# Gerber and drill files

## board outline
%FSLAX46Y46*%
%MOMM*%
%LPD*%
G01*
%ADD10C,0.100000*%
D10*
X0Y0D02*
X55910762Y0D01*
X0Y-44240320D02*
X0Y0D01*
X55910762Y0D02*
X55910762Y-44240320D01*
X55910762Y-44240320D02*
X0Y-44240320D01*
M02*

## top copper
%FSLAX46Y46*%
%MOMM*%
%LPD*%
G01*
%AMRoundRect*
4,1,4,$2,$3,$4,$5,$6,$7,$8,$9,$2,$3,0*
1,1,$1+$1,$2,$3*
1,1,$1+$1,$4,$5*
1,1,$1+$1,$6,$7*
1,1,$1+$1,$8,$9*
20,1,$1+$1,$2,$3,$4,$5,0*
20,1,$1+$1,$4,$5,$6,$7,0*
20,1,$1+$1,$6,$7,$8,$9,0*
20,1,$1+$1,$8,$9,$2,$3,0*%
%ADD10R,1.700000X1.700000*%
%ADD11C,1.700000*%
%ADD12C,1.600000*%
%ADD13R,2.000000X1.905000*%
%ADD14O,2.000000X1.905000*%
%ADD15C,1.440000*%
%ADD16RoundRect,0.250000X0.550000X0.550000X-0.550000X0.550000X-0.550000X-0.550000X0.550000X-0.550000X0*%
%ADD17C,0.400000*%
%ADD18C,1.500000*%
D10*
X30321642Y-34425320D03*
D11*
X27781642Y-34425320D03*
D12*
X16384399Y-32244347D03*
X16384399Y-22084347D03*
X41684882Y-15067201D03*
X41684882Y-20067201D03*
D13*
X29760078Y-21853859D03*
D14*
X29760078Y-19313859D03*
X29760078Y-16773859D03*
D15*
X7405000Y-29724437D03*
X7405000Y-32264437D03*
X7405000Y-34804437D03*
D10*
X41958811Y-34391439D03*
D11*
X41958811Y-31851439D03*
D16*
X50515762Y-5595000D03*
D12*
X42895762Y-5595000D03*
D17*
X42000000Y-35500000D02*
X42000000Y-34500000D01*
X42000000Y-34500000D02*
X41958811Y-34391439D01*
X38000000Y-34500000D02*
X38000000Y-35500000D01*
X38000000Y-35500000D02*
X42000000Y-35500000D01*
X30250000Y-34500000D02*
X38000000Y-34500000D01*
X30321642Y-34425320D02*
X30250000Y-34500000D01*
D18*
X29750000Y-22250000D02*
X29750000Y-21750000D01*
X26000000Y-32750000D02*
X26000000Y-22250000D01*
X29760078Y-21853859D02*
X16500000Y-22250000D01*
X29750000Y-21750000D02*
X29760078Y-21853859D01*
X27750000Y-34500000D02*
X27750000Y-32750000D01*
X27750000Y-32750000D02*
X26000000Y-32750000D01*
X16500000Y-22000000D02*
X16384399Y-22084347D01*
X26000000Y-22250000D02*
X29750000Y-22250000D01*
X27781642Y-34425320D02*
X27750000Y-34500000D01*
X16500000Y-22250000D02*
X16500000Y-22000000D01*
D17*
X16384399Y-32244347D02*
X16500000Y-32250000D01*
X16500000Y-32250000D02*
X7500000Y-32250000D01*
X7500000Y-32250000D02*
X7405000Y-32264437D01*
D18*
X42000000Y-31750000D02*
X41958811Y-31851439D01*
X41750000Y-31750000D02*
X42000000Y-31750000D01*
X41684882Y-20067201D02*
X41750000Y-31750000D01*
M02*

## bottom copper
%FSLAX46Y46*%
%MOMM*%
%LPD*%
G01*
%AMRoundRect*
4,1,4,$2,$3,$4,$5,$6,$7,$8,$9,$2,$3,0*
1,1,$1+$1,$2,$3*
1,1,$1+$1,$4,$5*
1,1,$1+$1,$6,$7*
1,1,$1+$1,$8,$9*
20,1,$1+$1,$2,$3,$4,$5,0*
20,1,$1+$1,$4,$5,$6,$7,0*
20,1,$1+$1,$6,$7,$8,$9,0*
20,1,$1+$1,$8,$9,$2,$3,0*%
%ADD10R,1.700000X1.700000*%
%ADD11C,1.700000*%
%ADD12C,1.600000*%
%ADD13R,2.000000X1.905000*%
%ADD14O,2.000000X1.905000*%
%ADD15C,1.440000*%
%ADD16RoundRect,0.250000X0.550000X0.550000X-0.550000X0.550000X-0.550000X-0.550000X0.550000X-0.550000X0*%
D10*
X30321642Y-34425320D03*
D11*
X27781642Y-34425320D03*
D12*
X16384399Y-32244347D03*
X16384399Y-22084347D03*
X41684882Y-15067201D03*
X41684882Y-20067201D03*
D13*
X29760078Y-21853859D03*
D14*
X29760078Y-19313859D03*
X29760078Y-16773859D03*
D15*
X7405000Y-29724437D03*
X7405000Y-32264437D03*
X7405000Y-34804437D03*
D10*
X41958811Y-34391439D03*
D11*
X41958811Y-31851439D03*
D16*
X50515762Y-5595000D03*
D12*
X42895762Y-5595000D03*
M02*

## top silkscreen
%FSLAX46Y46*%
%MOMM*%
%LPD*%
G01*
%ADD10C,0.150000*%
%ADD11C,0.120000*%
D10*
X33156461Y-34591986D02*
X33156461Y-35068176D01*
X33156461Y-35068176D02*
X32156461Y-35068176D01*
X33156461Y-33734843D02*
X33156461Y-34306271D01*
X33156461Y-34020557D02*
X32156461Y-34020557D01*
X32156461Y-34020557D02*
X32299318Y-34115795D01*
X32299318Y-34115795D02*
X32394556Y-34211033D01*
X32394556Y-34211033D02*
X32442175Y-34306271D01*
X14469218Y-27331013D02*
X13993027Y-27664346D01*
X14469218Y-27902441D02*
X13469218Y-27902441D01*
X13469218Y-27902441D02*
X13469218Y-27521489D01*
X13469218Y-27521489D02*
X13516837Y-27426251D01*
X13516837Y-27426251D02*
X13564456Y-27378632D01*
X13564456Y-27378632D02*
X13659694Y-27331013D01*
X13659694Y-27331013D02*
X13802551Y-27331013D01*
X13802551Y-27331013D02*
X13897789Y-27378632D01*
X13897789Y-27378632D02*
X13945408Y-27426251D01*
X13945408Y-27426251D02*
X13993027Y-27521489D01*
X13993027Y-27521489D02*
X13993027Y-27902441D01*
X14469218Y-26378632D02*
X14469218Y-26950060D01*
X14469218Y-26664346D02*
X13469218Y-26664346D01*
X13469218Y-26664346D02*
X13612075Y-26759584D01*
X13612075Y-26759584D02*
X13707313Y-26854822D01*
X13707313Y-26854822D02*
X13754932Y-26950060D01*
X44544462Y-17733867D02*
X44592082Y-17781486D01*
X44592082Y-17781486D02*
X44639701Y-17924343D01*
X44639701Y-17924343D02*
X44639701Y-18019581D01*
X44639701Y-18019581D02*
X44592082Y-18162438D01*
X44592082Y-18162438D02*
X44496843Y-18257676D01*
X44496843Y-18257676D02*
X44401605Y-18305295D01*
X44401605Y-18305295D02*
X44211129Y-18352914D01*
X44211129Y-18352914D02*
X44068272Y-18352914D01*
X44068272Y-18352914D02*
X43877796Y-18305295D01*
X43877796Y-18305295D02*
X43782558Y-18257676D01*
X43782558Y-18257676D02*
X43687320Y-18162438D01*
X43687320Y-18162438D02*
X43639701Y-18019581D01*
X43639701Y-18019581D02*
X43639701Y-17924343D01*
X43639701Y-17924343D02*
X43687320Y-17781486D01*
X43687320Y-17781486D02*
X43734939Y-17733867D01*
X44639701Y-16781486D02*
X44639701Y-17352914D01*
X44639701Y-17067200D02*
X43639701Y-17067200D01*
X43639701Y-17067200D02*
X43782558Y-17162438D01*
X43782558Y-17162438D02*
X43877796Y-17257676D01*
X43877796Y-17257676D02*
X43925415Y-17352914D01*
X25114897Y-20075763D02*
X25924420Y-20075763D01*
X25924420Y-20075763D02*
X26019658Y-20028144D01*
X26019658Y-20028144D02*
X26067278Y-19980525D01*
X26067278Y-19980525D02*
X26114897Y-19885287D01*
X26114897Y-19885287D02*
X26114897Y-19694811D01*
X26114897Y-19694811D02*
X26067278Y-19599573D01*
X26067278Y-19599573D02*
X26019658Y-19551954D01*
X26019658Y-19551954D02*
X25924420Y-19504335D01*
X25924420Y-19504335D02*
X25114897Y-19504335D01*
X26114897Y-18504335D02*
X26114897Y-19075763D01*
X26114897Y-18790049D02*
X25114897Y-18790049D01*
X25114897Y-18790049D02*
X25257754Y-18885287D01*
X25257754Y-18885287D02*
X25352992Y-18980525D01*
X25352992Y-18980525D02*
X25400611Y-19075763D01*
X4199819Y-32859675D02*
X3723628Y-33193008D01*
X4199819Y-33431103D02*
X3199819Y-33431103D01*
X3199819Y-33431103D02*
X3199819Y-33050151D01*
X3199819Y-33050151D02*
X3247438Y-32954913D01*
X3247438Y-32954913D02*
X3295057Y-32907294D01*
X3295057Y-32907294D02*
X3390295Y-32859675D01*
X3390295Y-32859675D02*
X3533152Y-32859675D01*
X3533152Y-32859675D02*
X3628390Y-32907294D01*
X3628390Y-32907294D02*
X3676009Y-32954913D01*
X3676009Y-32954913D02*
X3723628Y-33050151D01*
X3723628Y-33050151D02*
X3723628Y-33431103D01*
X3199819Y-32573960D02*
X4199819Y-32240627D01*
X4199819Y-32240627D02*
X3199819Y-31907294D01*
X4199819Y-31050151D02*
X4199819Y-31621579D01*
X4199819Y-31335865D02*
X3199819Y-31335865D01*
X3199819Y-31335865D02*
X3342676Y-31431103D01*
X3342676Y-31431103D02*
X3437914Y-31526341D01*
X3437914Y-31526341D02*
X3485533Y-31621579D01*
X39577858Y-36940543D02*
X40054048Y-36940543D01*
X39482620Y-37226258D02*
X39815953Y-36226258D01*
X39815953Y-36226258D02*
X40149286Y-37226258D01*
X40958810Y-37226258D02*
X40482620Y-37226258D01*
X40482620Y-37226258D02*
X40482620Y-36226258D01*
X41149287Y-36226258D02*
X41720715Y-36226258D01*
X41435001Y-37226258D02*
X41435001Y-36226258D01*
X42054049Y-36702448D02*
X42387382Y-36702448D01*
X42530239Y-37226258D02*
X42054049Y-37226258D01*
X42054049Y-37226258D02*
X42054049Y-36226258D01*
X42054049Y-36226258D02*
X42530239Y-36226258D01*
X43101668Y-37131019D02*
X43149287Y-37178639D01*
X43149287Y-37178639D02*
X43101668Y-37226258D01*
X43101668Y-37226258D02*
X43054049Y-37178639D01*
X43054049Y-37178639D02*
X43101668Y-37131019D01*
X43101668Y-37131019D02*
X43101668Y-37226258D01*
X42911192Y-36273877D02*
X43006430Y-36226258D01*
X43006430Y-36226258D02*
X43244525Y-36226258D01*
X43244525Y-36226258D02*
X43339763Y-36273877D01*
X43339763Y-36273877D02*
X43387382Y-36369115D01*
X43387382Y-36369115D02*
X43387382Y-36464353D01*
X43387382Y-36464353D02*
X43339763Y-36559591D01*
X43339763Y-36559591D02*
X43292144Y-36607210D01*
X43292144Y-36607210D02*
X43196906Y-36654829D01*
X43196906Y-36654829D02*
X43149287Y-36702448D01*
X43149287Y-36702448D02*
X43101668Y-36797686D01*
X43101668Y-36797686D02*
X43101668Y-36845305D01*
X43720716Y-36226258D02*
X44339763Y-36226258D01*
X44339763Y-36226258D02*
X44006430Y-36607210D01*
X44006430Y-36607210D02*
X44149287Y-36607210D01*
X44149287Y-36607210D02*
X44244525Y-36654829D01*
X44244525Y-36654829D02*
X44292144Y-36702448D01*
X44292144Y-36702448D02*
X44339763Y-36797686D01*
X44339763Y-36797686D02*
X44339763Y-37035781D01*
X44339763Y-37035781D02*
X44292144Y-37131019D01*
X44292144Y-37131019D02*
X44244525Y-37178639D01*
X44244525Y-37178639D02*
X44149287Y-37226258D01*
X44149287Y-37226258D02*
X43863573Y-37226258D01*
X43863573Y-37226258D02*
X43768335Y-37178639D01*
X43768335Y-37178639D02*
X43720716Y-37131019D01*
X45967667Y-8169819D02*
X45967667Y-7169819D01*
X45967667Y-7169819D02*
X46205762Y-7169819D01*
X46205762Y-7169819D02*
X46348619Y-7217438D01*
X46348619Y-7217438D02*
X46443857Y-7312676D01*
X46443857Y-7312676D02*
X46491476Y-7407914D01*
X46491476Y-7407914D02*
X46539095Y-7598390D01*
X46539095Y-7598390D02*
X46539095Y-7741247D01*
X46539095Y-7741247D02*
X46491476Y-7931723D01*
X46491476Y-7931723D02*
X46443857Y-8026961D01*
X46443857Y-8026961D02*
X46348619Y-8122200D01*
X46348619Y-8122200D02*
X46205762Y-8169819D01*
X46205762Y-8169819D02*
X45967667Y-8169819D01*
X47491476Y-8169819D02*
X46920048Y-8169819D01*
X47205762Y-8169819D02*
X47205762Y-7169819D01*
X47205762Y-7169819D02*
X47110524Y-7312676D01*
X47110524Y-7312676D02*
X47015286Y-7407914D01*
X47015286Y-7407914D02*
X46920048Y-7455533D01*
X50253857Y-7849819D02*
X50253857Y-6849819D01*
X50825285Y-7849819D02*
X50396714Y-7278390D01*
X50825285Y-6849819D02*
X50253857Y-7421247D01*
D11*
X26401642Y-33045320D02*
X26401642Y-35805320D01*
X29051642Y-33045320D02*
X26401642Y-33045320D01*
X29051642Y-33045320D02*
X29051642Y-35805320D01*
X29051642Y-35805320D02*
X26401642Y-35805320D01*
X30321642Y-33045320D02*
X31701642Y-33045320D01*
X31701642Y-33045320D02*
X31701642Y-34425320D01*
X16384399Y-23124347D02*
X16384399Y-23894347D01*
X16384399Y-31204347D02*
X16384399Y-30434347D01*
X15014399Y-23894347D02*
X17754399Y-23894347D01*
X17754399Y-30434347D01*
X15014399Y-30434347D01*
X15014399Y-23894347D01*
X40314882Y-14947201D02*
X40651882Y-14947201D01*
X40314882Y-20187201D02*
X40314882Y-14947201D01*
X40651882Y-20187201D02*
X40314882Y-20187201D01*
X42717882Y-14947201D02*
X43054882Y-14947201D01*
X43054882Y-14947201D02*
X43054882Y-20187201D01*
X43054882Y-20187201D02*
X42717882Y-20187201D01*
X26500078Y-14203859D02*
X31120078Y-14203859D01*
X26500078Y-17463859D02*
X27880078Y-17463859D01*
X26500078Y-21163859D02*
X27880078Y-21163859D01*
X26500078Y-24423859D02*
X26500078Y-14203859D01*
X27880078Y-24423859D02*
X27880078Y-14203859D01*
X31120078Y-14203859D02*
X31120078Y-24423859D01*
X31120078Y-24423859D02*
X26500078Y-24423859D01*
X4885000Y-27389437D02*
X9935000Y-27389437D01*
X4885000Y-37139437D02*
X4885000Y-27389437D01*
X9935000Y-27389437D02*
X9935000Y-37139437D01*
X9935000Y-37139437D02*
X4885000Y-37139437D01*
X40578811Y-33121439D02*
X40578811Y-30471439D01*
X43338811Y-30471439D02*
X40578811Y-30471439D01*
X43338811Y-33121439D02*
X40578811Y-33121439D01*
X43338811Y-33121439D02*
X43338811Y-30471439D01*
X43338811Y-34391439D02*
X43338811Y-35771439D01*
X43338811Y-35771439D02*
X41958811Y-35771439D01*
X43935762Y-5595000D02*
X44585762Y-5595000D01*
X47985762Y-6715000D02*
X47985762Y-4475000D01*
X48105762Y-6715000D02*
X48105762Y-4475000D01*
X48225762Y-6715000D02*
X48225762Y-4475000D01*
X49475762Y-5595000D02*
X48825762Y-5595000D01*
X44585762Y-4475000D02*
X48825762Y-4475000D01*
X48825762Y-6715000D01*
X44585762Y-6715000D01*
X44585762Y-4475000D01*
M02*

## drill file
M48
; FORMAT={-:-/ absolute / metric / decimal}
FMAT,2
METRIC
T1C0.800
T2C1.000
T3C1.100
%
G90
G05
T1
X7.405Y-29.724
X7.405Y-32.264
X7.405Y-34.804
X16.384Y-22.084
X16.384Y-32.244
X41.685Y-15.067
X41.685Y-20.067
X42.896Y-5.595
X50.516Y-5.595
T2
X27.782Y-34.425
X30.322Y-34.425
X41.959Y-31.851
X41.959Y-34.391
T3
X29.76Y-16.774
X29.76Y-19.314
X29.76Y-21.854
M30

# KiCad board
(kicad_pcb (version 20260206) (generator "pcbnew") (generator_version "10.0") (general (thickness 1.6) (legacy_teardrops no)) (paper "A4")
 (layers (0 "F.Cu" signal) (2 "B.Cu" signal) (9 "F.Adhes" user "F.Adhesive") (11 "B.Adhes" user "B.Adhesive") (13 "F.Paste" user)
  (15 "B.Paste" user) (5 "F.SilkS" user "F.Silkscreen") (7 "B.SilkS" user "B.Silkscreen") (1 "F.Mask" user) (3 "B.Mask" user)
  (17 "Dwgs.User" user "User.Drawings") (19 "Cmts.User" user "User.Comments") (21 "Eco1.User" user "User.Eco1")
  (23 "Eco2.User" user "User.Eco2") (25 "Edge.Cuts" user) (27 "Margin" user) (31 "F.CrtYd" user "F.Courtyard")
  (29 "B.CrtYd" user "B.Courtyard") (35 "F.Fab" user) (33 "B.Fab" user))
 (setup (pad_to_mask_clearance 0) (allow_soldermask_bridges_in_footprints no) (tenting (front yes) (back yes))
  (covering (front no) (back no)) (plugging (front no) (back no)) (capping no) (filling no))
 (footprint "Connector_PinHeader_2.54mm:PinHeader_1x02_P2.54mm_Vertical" (layer "F.Cu") (at 30.321642 34.42532 -90)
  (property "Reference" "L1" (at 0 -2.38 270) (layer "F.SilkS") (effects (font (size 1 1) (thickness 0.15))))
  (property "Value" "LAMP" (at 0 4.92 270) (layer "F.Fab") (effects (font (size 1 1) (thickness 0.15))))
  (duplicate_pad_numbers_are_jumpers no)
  (fp_line (start -1.38 3.92) (end 1.38 3.92) (stroke (width 0.12) (type solid)) (layer "F.SilkS"))
  (fp_line (start -1.38 1.27) (end -1.38 3.92) (stroke (width 0.12) (type solid)) (layer "F.SilkS"))
  (fp_line (start -1.38 1.27) (end 1.38 1.27) (stroke (width 0.12) (type solid)) (layer "F.SilkS"))
  (fp_line (start 1.38 1.27) (end 1.38 3.92) (stroke (width 0.12) (type solid)) (layer "F.SilkS"))
  (fp_line (start -1.38 0) (end -1.38 -1.38) (stroke (width 0.12) (type solid)) (layer "F.SilkS"))
  (fp_line (start -1.38 -1.38) (end 0 -1.38) (stroke (width 0.12) (type solid)) (layer "F.SilkS"))
  (pad "1" thru_hole rect (at 0 0 270) (size 1.7 1.7) (drill 1) (layers "*.Cu" "*.Mask") (remove_unused_layers no) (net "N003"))
  (pad "2" thru_hole circle (at 0 2.54 270) (size 1.7 1.7) (drill 1) (layers "*.Cu" "*.Mask") (remove_unused_layers no) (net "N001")))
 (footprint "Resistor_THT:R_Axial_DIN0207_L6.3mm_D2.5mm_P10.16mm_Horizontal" (layer "F.Cu") (at 16.384399 32.244347 90)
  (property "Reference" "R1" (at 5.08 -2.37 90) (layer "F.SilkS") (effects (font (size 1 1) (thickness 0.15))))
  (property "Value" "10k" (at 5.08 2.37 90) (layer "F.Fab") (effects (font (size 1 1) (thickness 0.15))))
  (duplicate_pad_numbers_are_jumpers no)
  (fp_line (start 9.12 0) (end 8.35 0) (stroke (width 0.12) (type solid)) (layer "F.SilkS"))
  (fp_line (start 1.04 0) (end 1.81 0) (stroke (width 0.12) (type solid)) (layer "F.SilkS"))
  (fp_rect (start 1.81 -1.37) (end 8.35 1.37) (stroke (width 0.12) (type solid)) (fill no) (layer "F.SilkS"))
  (pad "1" thru_hole circle (at 0 0 90) (size 1.6 1.6) (drill 0.8) (layers "*.Cu" "*.Mask") (remove_unused_layers no) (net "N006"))
  (pad "2" thru_hole circle (at 10.16 0 90) (size 1.6 1.6) (drill 0.8) (layers "*.Cu" "*.Mask") (remove_unused_layers no) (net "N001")))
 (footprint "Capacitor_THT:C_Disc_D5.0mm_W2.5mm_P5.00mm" (layer "F.Cu") (at 41.684882 15.067201 -90)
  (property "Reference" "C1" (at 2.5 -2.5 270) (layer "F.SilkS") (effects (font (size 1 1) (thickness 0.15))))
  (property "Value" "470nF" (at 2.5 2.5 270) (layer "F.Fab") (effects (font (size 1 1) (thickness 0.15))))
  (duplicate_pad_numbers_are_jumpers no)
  (fp_line (start -0.12 1.37) (end -0.12 1.033) (stroke (width 0.12) (type solid)) (layer "F.SilkS"))
  (fp_line (start 5.12 1.37) (end -0.12 1.37) (stroke (width 0.12) (type solid)) (layer "F.SilkS"))
  (fp_line (start 5.12 1.033) (end 5.12 1.37) (stroke (width 0.12) (type solid)) (layer "F.SilkS"))
  (fp_line (start -0.12 -1.033) (end -0.12 -1.37) (stroke (width 0.12) (type solid)) (layer "F.SilkS"))
  (fp_line (start -0.12 -1.37) (end 5.12 -1.37) (stroke (width 0.12) (type solid)) (layer "F.SilkS"))
  (fp_line (start 5.12 -1.37) (end 5.12 -1.033) (stroke (width 0.12) (type solid)) (layer "F.SilkS"))
  (pad "1" thru_hole circle (at 0 0 270) (size 1.6 1.6) (drill 0.8) (layers "*.Cu" "*.Mask") (remove_unused_layers no))
  (pad "2" thru_hole circle (at 5 0 270) (size 1.6 1.6) (drill 0.8) (layers "*.Cu" "*.Mask") (remove_unused_layers no) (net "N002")))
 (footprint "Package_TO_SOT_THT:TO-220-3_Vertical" (layer "F.Cu") (at 29.760078 21.853859 90)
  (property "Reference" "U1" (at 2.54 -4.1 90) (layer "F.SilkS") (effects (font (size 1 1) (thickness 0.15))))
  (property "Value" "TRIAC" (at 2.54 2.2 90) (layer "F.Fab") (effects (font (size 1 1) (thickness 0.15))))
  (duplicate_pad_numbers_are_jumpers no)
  (fp_line (start 7.65 -3.26) (end 7.65 1.36) (stroke (width 0.12) (type solid)) (layer "F.SilkS"))
  (fp_line (start 4.39 -3.26) (end 4.39 -1.88) (stroke (width 0.12) (type solid)) (layer "F.SilkS"))
  (fp_line (start 0.69 -3.26) (end 0.69 -1.88) (stroke (width 0.12) (type solid)) (layer "F.SilkS"))
  (fp_line (start -2.57 -3.26) (end 7.65 -3.26) (stroke (width 0.12) (type solid)) (layer "F.SilkS"))
  (fp_line (start -2.57 -1.88) (end 7.65 -1.88) (stroke (width 0.12) (type solid)) (layer "F.SilkS"))
  (fp_line (start 7.65 1.36) (end -2.57 1.36) (stroke (width 0.12) (type solid)) (layer "F.SilkS"))
  (fp_line (start -2.57 1.36) (end -2.57 -3.26) (stroke (width 0.12) (type solid)) (layer "F.SilkS"))
  (pad "1" thru_hole rect (at 0 0 90) (size 1.905 2) (drill 1.1) (layers "*.Cu" "*.Mask") (remove_unused_layers no) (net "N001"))
  (pad "2" thru_hole oval (at 2.54 0 90) (size 1.905 2) (drill 1.1) (layers "*.Cu" "*.Mask") (remove_unused_layers no) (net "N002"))
  (pad "3" thru_hole oval (at 5.08 0 90) (size 1.905 2) (drill 1.1) (layers "*.Cu" "*.Mask") (remove_unused_layers no) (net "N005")))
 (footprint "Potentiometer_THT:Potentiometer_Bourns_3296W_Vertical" (layer "F.Cu") (at 7.405 29.724437 90)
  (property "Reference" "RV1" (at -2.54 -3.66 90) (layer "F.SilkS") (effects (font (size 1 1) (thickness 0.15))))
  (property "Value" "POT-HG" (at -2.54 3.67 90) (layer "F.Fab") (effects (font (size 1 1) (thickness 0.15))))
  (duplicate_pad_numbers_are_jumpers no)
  (fp_line (start 2.335 -2.52) (end 2.335 2.53) (stroke (width 0.12) (type solid)) (layer "F.SilkS"))
  (fp_line (start -7.415 -2.52) (end 2.335 -2.52) (stroke (width 0.12) (type solid)) (layer "F.SilkS"))
  (fp_line (start 2.335 2.53) (end -7.415 2.53) (stroke (width 0.12) (type solid)) (layer "F.SilkS"))
  (fp_line (start -7.415 2.53) (end -7.415 -2.52) (stroke (width 0.12) (type solid)) (layer "F.SilkS"))
  (pad "1" thru_hole circle (at 0 0 90) (size 1.44 1.44) (drill 0.8) (layers "*.Cu" "*.Mask") (remove_unused_layers no) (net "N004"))
  (pad "2" thru_hole circle (at -2.54 0 90) (size 1.44 1.44) (drill 0.8) (layers "*.Cu" "*.Mask") (remove_unused_layers no) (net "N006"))
  (pad "3" thru_hole circle (at -5.08 0 90) (size 1.44 1.44) (drill 0.8) (layers "*.Cu" "*.Mask") (remove_unused_layers no)))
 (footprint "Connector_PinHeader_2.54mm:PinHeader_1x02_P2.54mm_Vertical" (layer "F.Cu") (at 41.958811 34.391439 180)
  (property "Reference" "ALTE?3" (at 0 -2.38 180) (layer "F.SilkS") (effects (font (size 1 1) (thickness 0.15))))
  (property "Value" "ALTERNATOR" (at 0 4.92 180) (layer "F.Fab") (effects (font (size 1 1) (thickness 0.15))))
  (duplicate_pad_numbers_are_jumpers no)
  (fp_line (start 1.38 1.27) (end 1.38 3.92) (stroke (width 0.12) (type solid)) (layer "F.SilkS"))
  (fp_line (start -1.38 3.92) (end 1.38 3.92) (stroke (width 0.12) (type solid)) (layer "F.SilkS"))
  (fp_line (start -1.38 1.27) (end 1.38 1.27) (stroke (width 0.12) (type solid)) (layer "F.SilkS"))
  (fp_line (start -1.38 1.27) (end -1.38 3.92) (stroke (width 0.12) (type solid)) (layer "F.SilkS"))
  (fp_line (start -1.38 0) (end -1.38 -1.38) (stroke (width 0.12) (type solid)) (layer "F.SilkS"))
  (fp_line (start -1.38 -1.38) (end 0 -1.38) (stroke (width 0.12) (type solid)) (layer "F.SilkS"))
  (pad "1" thru_hole rect (at 0 0 180) (size 1.7 1.7) (drill 1) (layers "*.Cu" "*.Mask") (remove_unused_layers no) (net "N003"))
  (pad "2" thru_hole circle (at 0 2.54 180) (size 1.7 1.7) (drill 1) (layers "*.Cu" "*.Mask") (remove_unused_layers no) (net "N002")))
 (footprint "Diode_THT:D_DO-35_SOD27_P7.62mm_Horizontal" (layer "F.Cu") (at 50.515762 5.595 180)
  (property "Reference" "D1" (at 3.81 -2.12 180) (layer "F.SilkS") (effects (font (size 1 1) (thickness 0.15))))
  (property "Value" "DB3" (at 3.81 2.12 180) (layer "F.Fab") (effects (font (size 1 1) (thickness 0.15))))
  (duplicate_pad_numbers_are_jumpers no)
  (fp_line (start 6.58 0) (end 5.93 0) (stroke (width 0.12) (type solid)) (layer "F.SilkS"))
  (fp_line (start 2.53 -1.12) (end 2.53 1.12) (stroke (width 0.12) (type solid)) (layer "F.SilkS"))
  (fp_line (start 2.41 -1.12) (end 2.41 1.12) (stroke (width 0.12) (type solid)) (layer "F.SilkS"))
  (fp_line (start 2.29 -1.12) (end 2.29 1.12) (stroke (width 0.12) (type solid)) (layer "F.SilkS"))
  (fp_line (start 1.04 0) (end 1.69 0) (stroke (width 0.12) (type solid)) (layer "F.SilkS"))
  (fp_rect (start 1.69 -1.12) (end 5.93 1.12) (stroke (width 0.12) (type solid)) (fill no) (layer "F.SilkS"))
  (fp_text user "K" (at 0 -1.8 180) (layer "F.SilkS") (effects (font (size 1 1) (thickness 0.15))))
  (pad "1" thru_hole roundrect (at 0 0 180) (size 1.6 1.6) (drill 0.8) (layers "*.Cu" "*.Mask") (remove_unused_layers no)
   (roundrect_rratio 0.15625))
  (pad "2" thru_hole circle (at 7.62 0 180) (size 1.6 1.6) (drill 0.8) (layers "*.Cu" "*.Mask") (remove_unused_layers no)))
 (gr_line (start 0 0) (end 55.910762 0) (stroke (width 0.1) (type default)) (layer "Edge.Cuts"))
 (gr_line (start 0 44.24032) (end 0 0) (stroke (width 0.1) (type default)) (layer "Edge.Cuts"))
 (gr_line (start 55.910762 0) (end 55.910762 44.24032) (stroke (width 0.1) (type default)) (layer "Edge.Cuts"))
 (gr_line (start 55.910762 44.24032) (end 0 44.24032) (stroke (width 0.1) (type default)) (layer "Edge.Cuts"))
 (segment (start 42 35.5) (end 42 34.5) (width 0.4) (layer "F.Cu") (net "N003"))
 (segment (start 42 34.5) (end 41.958811 34.391439) (width 0.4) (layer "F.Cu") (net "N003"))
 (segment (start 38 34.5) (end 38 35.5) (width 0.4) (layer "F.Cu") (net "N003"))
 (segment (start 38 35.5) (end 42 35.5) (width 0.4) (layer "F.Cu") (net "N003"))
 (segment (start 30.25 34.5) (end 38 34.5) (width 0.4) (layer "F.Cu") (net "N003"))
 (segment (start 30.321642 34.42532) (end 30.25 34.5) (width 0.4) (layer "F.Cu") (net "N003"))
 (segment (start 29.75 22.25) (end 29.75 21.75) (width 1.5) (layer "F.Cu") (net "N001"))
 (segment (start 26 32.75) (end 26 22.25) (width 1.5) (layer "F.Cu") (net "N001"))
 (segment (start 29.760078 21.853859) (end 16.5 22.25) (width 1.5) (layer "F.Cu") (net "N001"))
 (segment (start 29.75 21.75) (end 29.760078 21.853859) (width 1.5) (layer "F.Cu") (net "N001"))
 (segment (start 27.75 34.5) (end 27.75 32.75) (width 1.5) (layer "F.Cu") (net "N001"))
 (segment (start 27.75 32.75) (end 26 32.75) (width 1.5) (layer "F.Cu") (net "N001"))
 (segment (start 16.5 22) (end 16.384399 22.084347) (width 1.5) (layer "F.Cu") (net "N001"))
 (segment (start 26 22.25) (end 29.75 22.25) (width 1.5) (layer "F.Cu") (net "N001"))
 (segment (start 27.781642 34.42532) (end 27.75 34.5) (width 1.5) (layer "F.Cu") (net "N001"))
 (segment (start 16.5 22.25) (end 16.5 22) (width 1.5) (layer "F.Cu") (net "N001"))
 (segment (start 16.384399 32.244347) (end 16.5 32.25) (width 0.4) (layer "F.Cu") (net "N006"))
 (segment (start 16.5 32.25) (end 7.5 32.25) (width 0.4) (layer "F.Cu") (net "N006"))
 (segment (start 7.5 32.25) (end 7.405 32.264437) (width 0.4) (layer "F.Cu") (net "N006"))
 (segment (start 42 31.75) (end 41.958811 31.851439) (width 1.5) (layer "F.Cu") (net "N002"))
 (segment (start 41.75 31.75) (end 42 31.75) (width 1.5) (layer "F.Cu") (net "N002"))
 (segment (start 41.684882 20.067201) (end 41.75 31.75) (width 1.5) (layer "F.Cu") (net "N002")))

